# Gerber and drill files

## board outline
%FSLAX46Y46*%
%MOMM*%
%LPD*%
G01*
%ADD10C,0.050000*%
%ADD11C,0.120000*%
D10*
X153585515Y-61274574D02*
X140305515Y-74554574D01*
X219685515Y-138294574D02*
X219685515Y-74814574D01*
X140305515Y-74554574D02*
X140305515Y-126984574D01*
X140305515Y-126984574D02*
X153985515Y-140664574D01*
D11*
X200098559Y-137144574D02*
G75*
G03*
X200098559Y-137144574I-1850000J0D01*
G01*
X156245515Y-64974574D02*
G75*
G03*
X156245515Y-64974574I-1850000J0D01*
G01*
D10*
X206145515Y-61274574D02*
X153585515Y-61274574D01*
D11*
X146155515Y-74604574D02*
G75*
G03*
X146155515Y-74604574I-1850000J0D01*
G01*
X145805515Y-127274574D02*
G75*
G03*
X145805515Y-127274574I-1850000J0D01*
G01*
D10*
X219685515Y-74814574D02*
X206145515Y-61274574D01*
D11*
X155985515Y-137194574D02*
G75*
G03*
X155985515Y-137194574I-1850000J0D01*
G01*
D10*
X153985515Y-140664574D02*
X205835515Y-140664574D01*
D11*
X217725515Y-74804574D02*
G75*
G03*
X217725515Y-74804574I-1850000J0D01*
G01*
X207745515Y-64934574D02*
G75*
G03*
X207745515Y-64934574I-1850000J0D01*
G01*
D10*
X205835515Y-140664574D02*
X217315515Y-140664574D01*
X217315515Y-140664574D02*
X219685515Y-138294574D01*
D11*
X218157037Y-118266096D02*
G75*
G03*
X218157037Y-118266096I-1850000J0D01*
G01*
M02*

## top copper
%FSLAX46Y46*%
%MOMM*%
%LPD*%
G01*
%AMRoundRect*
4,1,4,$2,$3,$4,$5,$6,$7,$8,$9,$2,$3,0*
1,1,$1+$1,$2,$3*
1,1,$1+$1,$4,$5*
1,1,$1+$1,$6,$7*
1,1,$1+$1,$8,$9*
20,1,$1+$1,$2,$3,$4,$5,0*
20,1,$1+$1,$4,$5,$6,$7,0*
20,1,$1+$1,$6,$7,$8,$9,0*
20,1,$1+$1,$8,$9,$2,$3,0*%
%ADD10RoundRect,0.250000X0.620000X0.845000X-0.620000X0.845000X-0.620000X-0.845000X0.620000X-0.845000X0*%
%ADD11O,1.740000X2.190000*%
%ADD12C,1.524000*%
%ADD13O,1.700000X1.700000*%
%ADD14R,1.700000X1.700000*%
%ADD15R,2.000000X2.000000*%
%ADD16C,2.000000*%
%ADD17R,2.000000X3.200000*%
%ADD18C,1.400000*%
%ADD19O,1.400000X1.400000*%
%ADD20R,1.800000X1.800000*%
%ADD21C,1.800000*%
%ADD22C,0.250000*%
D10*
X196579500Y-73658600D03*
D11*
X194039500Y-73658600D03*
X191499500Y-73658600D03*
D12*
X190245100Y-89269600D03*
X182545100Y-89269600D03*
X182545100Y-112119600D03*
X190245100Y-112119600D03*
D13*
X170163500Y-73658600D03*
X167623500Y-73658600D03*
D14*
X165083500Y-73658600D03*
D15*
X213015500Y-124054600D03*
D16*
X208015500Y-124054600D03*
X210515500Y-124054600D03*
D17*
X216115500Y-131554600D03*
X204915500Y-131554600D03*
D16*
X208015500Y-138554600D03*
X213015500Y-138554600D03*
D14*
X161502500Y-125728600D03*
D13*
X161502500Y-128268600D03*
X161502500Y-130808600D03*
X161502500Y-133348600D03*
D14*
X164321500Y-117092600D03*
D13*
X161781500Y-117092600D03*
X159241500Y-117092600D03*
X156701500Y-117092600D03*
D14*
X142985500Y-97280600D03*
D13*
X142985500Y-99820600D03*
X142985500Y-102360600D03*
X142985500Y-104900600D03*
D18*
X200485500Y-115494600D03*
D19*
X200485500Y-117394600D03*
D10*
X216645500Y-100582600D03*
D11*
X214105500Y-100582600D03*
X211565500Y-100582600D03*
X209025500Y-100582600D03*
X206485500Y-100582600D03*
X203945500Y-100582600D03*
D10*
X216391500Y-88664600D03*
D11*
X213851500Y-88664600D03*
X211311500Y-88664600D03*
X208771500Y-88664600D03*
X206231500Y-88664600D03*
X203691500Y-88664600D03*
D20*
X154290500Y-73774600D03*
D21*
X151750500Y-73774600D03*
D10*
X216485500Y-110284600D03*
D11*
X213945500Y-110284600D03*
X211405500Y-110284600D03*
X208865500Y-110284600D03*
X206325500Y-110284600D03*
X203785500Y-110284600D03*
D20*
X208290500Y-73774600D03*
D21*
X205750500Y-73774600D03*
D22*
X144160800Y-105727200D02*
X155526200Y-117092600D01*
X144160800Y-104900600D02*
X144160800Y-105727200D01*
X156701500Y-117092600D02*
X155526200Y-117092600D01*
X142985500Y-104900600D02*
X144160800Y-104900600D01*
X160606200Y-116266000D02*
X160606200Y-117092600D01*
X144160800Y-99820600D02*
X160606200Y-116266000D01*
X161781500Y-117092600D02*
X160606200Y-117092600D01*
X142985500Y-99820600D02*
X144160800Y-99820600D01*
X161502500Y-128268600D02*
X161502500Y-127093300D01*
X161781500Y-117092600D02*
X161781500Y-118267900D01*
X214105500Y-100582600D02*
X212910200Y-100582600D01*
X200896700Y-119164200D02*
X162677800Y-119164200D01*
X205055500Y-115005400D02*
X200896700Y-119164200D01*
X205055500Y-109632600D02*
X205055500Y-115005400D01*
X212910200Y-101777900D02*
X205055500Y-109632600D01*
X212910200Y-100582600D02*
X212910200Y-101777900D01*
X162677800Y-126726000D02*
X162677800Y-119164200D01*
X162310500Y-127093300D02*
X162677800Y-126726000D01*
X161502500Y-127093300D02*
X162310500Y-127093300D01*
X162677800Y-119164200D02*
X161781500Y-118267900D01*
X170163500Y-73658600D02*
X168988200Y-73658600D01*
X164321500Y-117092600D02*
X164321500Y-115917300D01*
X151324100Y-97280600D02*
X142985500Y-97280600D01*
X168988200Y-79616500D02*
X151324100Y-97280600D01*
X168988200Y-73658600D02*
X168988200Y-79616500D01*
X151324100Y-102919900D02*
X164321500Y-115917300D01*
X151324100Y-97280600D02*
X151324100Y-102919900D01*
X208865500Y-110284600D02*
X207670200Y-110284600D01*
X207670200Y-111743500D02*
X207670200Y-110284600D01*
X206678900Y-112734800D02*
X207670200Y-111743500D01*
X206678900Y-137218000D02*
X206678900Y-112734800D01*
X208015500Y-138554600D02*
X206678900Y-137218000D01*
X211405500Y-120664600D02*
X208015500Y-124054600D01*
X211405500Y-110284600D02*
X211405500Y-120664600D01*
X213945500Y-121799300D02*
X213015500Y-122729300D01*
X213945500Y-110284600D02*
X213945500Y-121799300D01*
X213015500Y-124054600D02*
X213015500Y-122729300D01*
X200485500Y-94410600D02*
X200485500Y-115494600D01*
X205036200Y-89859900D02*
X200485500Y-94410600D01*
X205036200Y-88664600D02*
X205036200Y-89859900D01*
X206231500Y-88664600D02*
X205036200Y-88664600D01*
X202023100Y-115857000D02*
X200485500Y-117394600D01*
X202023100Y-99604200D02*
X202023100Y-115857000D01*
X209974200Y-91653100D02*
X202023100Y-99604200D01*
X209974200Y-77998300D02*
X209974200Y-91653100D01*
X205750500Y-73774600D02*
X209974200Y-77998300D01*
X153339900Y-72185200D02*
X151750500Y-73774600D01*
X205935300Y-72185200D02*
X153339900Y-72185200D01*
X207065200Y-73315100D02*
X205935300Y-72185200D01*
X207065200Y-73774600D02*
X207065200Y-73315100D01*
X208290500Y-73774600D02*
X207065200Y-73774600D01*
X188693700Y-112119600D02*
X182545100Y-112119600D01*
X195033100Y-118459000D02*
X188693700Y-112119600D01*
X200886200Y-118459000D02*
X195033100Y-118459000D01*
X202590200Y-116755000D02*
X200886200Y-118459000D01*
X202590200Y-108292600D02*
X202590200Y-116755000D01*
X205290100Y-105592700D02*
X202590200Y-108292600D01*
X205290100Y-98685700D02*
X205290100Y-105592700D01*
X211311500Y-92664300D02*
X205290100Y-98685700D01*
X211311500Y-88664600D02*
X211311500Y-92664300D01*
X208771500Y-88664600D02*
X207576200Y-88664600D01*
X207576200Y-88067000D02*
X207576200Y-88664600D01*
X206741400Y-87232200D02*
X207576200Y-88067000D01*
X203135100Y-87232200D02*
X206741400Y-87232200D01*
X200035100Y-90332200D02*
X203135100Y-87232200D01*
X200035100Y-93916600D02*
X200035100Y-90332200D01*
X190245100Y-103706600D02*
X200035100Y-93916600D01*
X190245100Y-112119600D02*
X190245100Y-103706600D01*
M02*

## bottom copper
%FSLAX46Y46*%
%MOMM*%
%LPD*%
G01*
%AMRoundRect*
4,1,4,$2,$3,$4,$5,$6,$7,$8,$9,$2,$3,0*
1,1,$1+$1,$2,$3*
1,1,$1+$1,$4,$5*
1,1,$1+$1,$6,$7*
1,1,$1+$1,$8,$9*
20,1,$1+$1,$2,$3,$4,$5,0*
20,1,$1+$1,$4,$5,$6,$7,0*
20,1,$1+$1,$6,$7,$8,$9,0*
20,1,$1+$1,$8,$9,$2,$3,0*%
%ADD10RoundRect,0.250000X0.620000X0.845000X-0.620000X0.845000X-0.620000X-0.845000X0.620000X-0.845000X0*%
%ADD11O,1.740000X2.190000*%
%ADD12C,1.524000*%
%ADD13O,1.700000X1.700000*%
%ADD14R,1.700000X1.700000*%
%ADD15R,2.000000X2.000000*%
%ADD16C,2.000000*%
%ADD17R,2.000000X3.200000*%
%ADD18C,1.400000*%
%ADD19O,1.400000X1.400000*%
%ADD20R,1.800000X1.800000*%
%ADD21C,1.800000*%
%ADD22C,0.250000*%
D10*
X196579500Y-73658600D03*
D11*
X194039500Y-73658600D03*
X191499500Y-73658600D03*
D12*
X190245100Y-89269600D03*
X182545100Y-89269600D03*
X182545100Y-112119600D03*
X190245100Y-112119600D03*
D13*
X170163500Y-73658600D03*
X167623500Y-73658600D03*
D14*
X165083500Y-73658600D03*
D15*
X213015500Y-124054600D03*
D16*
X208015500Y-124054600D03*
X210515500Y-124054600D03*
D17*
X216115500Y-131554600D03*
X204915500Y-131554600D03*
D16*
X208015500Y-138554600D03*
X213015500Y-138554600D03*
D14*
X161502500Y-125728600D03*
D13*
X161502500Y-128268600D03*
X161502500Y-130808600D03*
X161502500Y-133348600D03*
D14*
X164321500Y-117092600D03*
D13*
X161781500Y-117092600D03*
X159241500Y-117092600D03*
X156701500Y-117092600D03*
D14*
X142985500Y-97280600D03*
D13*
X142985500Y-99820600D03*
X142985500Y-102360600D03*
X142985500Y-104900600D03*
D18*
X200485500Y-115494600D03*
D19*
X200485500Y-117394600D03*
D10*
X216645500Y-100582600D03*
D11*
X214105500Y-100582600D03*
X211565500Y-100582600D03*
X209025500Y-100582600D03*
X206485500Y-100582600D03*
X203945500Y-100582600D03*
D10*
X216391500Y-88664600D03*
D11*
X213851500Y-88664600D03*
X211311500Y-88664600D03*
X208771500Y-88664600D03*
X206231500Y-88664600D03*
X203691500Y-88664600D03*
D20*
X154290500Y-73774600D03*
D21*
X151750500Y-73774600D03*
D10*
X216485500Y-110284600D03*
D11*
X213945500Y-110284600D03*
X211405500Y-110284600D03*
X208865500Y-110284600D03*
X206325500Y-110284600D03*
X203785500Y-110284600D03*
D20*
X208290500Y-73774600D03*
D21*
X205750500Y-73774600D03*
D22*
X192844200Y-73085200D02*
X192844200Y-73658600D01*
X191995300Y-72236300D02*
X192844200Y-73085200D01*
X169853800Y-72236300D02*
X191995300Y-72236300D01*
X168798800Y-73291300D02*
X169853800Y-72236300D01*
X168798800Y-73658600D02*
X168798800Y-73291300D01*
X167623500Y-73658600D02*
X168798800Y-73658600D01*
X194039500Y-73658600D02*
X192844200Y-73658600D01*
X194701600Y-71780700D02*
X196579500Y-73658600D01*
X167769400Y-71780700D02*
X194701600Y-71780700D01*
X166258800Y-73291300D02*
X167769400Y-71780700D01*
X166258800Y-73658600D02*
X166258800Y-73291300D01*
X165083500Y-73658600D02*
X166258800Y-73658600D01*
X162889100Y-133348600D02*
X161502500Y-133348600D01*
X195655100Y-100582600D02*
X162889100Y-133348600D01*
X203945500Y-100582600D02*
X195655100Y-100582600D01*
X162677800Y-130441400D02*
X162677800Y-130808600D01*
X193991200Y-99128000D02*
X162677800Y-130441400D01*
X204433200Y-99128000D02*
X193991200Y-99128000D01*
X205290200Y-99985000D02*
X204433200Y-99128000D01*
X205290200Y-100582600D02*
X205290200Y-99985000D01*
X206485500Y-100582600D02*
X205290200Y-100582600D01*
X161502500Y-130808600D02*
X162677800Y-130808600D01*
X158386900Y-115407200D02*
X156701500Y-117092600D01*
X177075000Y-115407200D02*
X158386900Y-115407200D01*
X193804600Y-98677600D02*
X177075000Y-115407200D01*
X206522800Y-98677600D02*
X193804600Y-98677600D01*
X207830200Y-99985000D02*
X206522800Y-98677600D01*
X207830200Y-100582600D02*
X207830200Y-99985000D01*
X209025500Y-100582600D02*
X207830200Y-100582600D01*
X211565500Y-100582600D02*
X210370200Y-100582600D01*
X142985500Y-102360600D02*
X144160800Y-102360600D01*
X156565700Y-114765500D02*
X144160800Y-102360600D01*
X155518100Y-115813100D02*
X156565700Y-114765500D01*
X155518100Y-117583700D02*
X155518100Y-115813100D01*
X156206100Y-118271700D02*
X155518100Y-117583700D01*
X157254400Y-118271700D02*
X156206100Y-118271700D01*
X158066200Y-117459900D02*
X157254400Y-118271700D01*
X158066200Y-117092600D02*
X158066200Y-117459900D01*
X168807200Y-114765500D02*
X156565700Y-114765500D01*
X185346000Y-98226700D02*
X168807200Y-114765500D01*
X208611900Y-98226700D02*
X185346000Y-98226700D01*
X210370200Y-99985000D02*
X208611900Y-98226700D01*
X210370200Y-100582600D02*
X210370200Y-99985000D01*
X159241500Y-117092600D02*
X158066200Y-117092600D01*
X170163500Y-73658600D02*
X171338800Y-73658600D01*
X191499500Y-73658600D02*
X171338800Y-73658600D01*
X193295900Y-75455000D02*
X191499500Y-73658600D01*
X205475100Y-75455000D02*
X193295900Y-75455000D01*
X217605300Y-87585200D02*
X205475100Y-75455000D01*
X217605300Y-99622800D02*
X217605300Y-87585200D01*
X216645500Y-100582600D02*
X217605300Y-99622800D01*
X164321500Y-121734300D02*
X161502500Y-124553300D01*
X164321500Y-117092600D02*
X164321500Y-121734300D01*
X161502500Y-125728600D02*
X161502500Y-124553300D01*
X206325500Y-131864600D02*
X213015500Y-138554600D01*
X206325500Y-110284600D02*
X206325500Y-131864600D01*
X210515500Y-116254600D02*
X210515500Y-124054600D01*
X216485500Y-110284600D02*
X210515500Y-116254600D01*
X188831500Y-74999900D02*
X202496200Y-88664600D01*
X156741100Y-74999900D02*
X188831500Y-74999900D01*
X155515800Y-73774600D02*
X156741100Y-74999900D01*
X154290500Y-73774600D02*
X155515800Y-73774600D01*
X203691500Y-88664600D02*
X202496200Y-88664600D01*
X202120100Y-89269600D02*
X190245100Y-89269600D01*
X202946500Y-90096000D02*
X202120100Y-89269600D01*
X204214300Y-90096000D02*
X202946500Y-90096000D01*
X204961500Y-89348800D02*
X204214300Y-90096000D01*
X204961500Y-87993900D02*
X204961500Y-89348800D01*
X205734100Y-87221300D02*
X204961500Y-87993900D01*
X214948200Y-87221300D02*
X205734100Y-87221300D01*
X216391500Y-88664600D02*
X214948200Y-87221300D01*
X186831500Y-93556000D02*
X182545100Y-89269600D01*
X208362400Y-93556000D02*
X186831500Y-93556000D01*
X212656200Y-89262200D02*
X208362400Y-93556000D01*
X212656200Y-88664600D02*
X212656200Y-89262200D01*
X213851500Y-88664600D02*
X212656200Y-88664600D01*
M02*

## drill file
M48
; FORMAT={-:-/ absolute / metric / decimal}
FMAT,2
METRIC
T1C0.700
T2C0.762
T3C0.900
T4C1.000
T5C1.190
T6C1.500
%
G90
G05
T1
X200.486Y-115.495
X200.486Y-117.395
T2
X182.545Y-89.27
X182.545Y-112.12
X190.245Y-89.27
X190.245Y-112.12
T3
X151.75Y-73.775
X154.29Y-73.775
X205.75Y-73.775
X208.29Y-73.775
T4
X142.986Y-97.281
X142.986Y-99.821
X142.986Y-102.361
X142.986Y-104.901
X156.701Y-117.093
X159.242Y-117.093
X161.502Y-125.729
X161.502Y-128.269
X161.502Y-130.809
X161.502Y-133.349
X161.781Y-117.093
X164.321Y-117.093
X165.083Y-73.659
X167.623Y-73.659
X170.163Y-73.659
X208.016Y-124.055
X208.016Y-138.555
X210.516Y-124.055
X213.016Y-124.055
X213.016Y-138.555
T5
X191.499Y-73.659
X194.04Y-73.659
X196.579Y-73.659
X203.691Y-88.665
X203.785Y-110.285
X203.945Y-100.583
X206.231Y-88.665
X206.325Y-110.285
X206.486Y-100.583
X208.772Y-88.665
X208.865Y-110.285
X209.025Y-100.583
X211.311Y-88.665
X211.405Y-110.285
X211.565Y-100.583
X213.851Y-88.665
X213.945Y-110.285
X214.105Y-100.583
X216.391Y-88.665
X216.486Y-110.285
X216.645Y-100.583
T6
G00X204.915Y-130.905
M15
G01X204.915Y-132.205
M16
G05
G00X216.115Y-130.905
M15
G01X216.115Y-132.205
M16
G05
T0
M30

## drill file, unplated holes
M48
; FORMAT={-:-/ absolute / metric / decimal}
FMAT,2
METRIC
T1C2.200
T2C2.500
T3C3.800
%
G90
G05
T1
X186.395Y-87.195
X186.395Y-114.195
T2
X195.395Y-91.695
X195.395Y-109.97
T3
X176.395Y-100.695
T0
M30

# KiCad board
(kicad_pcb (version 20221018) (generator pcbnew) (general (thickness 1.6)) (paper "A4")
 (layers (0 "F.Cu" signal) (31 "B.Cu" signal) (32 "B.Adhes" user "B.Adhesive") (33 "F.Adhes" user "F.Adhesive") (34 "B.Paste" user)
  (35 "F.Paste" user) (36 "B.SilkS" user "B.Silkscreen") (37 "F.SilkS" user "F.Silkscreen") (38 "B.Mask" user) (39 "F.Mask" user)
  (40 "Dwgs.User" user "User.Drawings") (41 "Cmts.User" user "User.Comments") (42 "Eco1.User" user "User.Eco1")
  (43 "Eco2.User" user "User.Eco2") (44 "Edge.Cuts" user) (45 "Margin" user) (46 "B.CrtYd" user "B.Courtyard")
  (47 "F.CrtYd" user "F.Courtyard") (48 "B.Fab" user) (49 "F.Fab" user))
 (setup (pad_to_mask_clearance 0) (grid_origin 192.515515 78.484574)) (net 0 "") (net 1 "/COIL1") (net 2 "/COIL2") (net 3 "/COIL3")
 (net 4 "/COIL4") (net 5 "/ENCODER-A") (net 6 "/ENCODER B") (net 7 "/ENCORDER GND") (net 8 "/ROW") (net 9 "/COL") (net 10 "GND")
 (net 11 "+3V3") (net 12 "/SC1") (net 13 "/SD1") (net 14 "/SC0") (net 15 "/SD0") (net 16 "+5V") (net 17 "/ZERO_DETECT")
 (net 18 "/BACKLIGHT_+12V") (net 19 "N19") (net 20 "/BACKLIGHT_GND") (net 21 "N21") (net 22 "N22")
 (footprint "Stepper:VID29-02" (layer "F.Cu") (at 186.3951 100.8596 -90)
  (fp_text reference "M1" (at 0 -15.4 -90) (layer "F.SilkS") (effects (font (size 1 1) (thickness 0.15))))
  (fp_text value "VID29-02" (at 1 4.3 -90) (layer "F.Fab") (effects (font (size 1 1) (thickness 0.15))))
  (pad "" np_thru_hole circle (at -13.665 0 270) (size 2.2 2.2) (drill 2.2) (layers "*.Cu" "*.Mask"))
  (pad "" np_thru_hole circle (at -9.165 -9 270) (size 2.5 2.5) (drill 2.5) (layers "*.Cu" "*.Mask"))
  (pad "" np_thru_hole circle (at -0.165 10 270) (size 3.8 3.8) (drill 3.8) (layers "*.Cu" "*.Mask"))
  (pad "" np_thru_hole circle (at 9.11 -9 270) (size 2.5 2.5) (drill 2.5) (layers "*.Cu" "*.Mask"))
  (pad "" np_thru_hole circle (at 13.335 0 270) (size 2.2 2.2) (drill 2.2) (layers "*.Cu" "*.Mask"))
  (pad "1" thru_hole circle (at -11.59 -3.85 270) (size 1.524 1.524) (drill 0.762) (layers "*.Cu" "*.Mask") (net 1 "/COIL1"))
  (pad "2" thru_hole circle (at -11.59 3.85 270) (size 1.524 1.524) (drill 0.762) (layers "*.Cu" "*.Mask") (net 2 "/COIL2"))
  (pad "3" thru_hole circle (at 11.26 3.85 270) (size 1.524 1.524) (drill 0.762) (layers "*.Cu" "*.Mask") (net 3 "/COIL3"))
  (pad "4" thru_hole circle (at 11.26 -3.85 270) (size 1.524 1.524) (drill 0.762) (layers "*.Cu" "*.Mask") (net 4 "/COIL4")))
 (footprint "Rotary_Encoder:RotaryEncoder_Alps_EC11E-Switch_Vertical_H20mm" (layer "F.Cu") (at 213.0155 124.0546 -90)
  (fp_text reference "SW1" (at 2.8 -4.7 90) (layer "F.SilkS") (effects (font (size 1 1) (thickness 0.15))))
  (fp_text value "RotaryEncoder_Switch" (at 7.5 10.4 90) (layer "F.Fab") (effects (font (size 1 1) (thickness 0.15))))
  (pad "A" thru_hole rect (at 0 0 270) (size 2 2) (drill 1) (layers "*.Cu" "*.Mask") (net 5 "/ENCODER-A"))
  (pad "B" thru_hole circle (at 0 5 270) (size 2 2) (drill 1) (layers "*.Cu" "*.Mask") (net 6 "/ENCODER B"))
  (pad "C" thru_hole circle (at 0 2.5 270) (size 2 2) (drill 1) (layers "*.Cu" "*.Mask") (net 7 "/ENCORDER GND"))
  (pad "MP" thru_hole rect (at 7.5 -3.1 270) (size 3.2 2) (drill oval 2.8 1.5) (layers "*.Cu" "*.Mask"))
  (pad "MP" thru_hole rect (at 7.5 8.1 270) (size 3.2 2) (drill oval 2.8 1.5) (layers "*.Cu" "*.Mask"))
  (pad "S1" thru_hole circle (at 14.5 5 270) (size 2 2) (drill 1) (layers "*.Cu" "*.Mask") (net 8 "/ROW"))
  (pad "S2" thru_hole circle (at 14.5 0 270) (size 2 2) (drill 1) (layers "*.Cu" "*.Mask") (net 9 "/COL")))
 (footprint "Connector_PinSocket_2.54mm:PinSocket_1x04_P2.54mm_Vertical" (layer "F.Cu") (at 161.5025 125.7286)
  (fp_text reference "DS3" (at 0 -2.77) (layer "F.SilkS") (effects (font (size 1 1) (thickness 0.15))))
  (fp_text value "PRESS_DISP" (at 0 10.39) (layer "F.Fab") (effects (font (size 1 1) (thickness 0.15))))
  (pad "1" thru_hole rect (at 0 0) (size 1.7 1.7) (drill 1) (layers "*.Cu" "*.Mask") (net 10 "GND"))
  (pad "2" thru_hole oval (at 0 2.54) (size 1.7 1.7) (drill 1) (layers "*.Cu" "*.Mask") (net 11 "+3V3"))
  (pad "3" thru_hole oval (at 0 5.08) (size 1.7 1.7) (drill 1) (layers "*.Cu" "*.Mask") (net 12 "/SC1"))
  (pad "4" thru_hole oval (at 0 7.62) (size 1.7 1.7) (drill 1) (layers "*.Cu" "*.Mask") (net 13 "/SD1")))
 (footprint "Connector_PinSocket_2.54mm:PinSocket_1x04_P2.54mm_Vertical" (layer "F.Cu") (at 164.3215 117.0926 -90)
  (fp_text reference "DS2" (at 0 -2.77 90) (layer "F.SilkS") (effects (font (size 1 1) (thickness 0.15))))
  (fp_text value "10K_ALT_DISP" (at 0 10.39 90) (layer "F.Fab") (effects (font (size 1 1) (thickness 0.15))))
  (pad "1" thru_hole rect (at 0 0 270) (size 1.7 1.7) (drill 1) (layers "*.Cu" "*.Mask") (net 10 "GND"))
  (pad "2" thru_hole oval (at 0 2.54 270) (size 1.7 1.7) (drill 1) (layers "*.Cu" "*.Mask") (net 11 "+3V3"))
  (pad "3" thru_hole oval (at 0 5.08 270) (size 1.7 1.7) (drill 1) (layers "*.Cu" "*.Mask") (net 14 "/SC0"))
  (pad "4" thru_hole oval (at 0 7.62 270) (size 1.7 1.7) (drill 1) (layers "*.Cu" "*.Mask") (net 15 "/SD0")))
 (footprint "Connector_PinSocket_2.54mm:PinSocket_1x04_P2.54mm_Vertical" (layer "F.Cu") (at 142.9855 97.2806)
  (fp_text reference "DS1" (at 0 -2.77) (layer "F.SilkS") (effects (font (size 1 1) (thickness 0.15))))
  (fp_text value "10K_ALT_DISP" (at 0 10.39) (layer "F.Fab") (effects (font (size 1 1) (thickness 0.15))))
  (pad "1" thru_hole rect (at 0 0) (size 1.7 1.7) (drill 1) (layers "*.Cu" "*.Mask") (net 10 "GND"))
  (pad "2" thru_hole oval (at 0 2.54) (size 1.7 1.7) (drill 1) (layers "*.Cu" "*.Mask") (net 11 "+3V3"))
  (pad "3" thru_hole oval (at 0 5.08) (size 1.7 1.7) (drill 1) (layers "*.Cu" "*.Mask") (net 14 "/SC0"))
  (pad "4" thru_hole oval (at 0 7.62) (size 1.7 1.7) (drill 1) (layers "*.Cu" "*.Mask") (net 15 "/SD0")))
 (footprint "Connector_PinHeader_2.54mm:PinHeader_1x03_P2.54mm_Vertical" (layer "B.Cu") (at 165.0835 73.6586 -90)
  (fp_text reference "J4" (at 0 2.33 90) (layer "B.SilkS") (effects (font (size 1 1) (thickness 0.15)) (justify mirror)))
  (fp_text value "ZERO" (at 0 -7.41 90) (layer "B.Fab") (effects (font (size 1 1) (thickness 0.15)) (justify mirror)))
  (pad "1" thru_hole rect (at 0 0 270) (size 1.7 1.7) (drill 1) (layers "*.Cu" "*.Mask") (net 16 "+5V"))
  (pad "2" thru_hole oval (at 0 -2.54 270) (size 1.7 1.7) (drill 1) (layers "*.Cu" "*.Mask") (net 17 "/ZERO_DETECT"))
  (pad "3" thru_hole oval (at 0 -5.08 270) (size 1.7 1.7) (drill 1) (layers "*.Cu" "*.Mask") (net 10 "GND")))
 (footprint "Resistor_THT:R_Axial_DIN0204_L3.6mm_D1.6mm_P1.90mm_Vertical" (layer "B.Cu") (at 200.4855 115.4946 -90)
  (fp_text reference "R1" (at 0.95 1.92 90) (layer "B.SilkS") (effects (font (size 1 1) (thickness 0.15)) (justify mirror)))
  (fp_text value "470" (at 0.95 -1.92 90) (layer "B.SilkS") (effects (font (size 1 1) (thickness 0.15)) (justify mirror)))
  (pad "1" thru_hole circle (at 0 0 270) (size 1.4 1.4) (drill 0.7) (layers "*.Cu" "*.Mask") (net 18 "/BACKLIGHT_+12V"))
  (pad "2" thru_hole oval (at 1.9 0 270) (size 1.4 1.4) (drill 0.7) (layers "*.Cu" "*.Mask") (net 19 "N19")))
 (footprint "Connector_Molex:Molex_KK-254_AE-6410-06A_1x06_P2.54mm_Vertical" (layer "B.Cu") (at 216.6455 100.5826 180)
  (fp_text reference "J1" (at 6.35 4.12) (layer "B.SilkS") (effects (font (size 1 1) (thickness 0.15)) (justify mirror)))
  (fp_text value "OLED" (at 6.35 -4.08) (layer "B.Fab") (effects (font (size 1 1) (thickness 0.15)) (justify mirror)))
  (pad "1" thru_hole roundrect (at 0 0 180) (size 1.74 2.19) (drill 1.19) (layers "*.Cu" "*.Mask") (roundrect_rratio 0.1436781609)
   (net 10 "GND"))
  (pad "2" thru_hole oval (at 2.54 0 180) (size 1.74 2.19) (drill 1.19) (layers "*.Cu" "*.Mask") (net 11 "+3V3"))
  (pad "3" thru_hole oval (at 5.08 0 180) (size 1.74 2.19) (drill 1.19) (layers "*.Cu" "*.Mask") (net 14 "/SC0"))
  (pad "4" thru_hole oval (at 7.62 0 180) (size 1.74 2.19) (drill 1.19) (layers "*.Cu" "*.Mask") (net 15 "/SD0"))
  (pad "5" thru_hole oval (at 10.16 0 180) (size 1.74 2.19) (drill 1.19) (layers "*.Cu" "*.Mask") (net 12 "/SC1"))
  (pad "6" thru_hole oval (at 12.7 0 180) (size 1.74 2.19) (drill 1.19) (layers "*.Cu" "*.Mask") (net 13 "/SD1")))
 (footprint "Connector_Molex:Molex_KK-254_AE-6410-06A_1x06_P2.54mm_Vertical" (layer "B.Cu") (at 216.3915 88.6646 180)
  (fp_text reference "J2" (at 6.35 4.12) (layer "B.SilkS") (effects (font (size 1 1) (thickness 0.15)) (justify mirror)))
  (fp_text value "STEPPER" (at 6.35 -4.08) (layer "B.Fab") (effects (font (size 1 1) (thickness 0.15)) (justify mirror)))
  (pad "1" thru_hole roundrect (at 0 0 180) (size 1.74 2.19) (drill 1.19) (layers "*.Cu" "*.Mask") (roundrect_rratio 0.1436781609)
   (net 1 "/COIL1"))
  (pad "2" thru_hole oval (at 2.54 0 180) (size 1.74 2.19) (drill 1.19) (layers "*.Cu" "*.Mask") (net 2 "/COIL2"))
  (pad "3" thru_hole oval (at 5.08 0 180) (size 1.74 2.19) (drill 1.19) (layers "*.Cu" "*.Mask") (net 3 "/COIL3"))
  (pad "4" thru_hole oval (at 7.62 0 180) (size 1.74 2.19) (drill 1.19) (layers "*.Cu" "*.Mask") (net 4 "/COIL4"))
  (pad "5" thru_hole oval (at 10.16 0 180) (size 1.74 2.19) (drill 1.19) (layers "*.Cu" "*.Mask") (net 18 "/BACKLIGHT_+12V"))
  (pad "6" thru_hole oval (at 12.7 0 180) (size 1.74 2.19) (drill 1.19) (layers "*.Cu" "*.Mask") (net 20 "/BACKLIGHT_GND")))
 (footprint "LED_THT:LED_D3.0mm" (layer "B.Cu") (at 154.2905 73.7746 180)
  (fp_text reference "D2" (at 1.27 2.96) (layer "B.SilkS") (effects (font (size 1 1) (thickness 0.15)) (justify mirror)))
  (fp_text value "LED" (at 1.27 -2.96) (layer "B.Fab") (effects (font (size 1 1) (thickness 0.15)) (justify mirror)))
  (pad "1" thru_hole rect (at 0 0 180) (size 1.8 1.8) (drill 0.9) (layers "*.Cu" "*.Mask") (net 20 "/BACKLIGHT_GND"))
  (pad "2" thru_hole circle (at 2.54 0 180) (size 1.8 1.8) (drill 0.9) (layers "*.Cu" "*.Mask") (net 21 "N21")))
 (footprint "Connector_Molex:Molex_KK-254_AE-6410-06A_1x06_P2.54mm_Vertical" (layer "B.Cu") (at 216.4855 110.2846 180)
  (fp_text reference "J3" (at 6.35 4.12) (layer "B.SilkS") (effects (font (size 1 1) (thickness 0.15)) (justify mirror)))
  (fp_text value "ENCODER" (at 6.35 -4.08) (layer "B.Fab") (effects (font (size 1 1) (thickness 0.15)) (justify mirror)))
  (pad "1" thru_hole roundrect (at 0 0 180) (size 1.74 2.19) (drill 1.19) (layers "*.Cu" "*.Mask") (roundrect_rratio 0.1436781609)
   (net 7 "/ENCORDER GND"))
  (pad "2" thru_hole oval (at 2.54 0 180) (size 1.74 2.19) (drill 1.19) (layers "*.Cu" "*.Mask") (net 5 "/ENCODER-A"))
  (pad "3" thru_hole oval (at 5.08 0 180) (size 1.74 2.19) (drill 1.19) (layers "*.Cu" "*.Mask") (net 6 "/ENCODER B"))
  (pad "4" thru_hole oval (at 7.62 0 180) (size 1.74 2.19) (drill 1.19) (layers "*.Cu" "*.Mask") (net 8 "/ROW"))
  (pad "5" thru_hole oval (at 10.16 0 180) (size 1.74 2.19) (drill 1.19) (layers "*.Cu" "*.Mask") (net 9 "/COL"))
  (pad "6" thru_hole oval (at 12.7 0 180) (size 1.74 2.19) (drill 1.19) (layers "*.Cu" "*.Mask") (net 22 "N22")))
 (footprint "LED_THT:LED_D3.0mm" (layer "B.Cu") (at 208.2905 73.7746 180)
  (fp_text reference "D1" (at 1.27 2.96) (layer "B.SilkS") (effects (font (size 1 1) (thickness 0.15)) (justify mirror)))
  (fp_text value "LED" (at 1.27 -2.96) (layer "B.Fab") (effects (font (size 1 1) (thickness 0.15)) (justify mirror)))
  (pad "1" thru_hole rect (at 0 0 180) (size 1.8 1.8) (drill 0.9) (layers "*.Cu" "*.Mask") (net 21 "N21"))
  (pad "2" thru_hole circle (at 2.54 0 180) (size 1.8 1.8) (drill 0.9) (layers "*.Cu" "*.Mask") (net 19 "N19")))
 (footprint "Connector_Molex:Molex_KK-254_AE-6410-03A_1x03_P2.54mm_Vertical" (layer "B.Cu") (at 196.5795 73.6586 180)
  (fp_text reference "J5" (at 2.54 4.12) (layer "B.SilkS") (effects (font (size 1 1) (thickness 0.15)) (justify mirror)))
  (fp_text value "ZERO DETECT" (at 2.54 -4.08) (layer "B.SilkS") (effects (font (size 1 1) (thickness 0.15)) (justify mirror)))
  (pad "1" thru_hole roundrect (at 0 0 180) (size 1.74 2.19) (drill 1.19) (layers "*.Cu" "*.Mask") (roundrect_rratio 0.1436781609)
   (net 16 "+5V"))
  (pad "2" thru_hole oval (at 2.54 0 180) (size 1.74 2.19) (drill 1.19) (layers "*.Cu" "*.Mask") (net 17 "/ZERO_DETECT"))
  (pad "3" thru_hole oval (at 5.08 0 180) (size 1.74 2.19) (drill 1.19) (layers "*.Cu" "*.Mask") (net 10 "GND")))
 (gr_line (start 153.585515 61.274574) (end 140.305515 74.554574) (stroke (width 0.05) (type solid)) (layer "Edge.Cuts"))
 (gr_line (start 219.685515 138.294574) (end 219.685515 74.814574) (stroke (width 0.05) (type solid)) (layer "Edge.Cuts"))
 (gr_line (start 140.305515 74.554574) (end 140.305515 126.984574) (stroke (width 0.05) (type solid)) (layer "Edge.Cuts"))
 (gr_line (start 140.305515 126.984574) (end 153.985515 140.664574) (stroke (width 0.05) (type solid)) (layer "Edge.Cuts"))
 (gr_circle (center 198.248559 137.144574) (end 200.098559 137.144574) (stroke (width 0.12) (type solid)) (fill none) (layer "Edge.Cuts"))
 (gr_circle (center 154.395515 64.974574) (end 156.245515 64.974574) (stroke (width 0.12) (type solid)) (fill none) (layer "Edge.Cuts"))
 (gr_line (start 206.145515 61.274574) (end 153.585515 61.274574) (stroke (width 0.05) (type solid)) (layer "Edge.Cuts"))
 (gr_circle (center 144.305515 74.604574) (end 146.155515 74.604574) (stroke (width 0.12) (type solid)) (fill none) (layer "Edge.Cuts"))
 (gr_circle (center 143.955515 127.274574) (end 145.805515 127.274574) (stroke (width 0.12) (type solid)) (fill none) (layer "Edge.Cuts"))
 (gr_line (start 219.685515 74.814574) (end 206.145515 61.274574) (stroke (width 0.05) (type solid)) (layer "Edge.Cuts"))
 (gr_circle (center 154.135515 137.194574) (end 155.985515 137.194574) (stroke (width 0.12) (type solid)) (fill none) (layer "Edge.Cuts"))
 (gr_line (start 153.985515 140.664574) (end 205.835515 140.664574) (stroke (width 0.05) (type solid)) (layer "Edge.Cuts"))
 (gr_circle (center 215.875515 74.804574) (end 217.725515 74.804574) (stroke (width 0.12) (type solid)) (fill none) (layer "Edge.Cuts"))
 (gr_circle (center 205.895515 64.934574) (end 207.745515 64.934574) (stroke (width 0.12) (type solid)) (fill none) (layer "Edge.Cuts"))
 (gr_line (start 205.835515 140.664574) (end 217.315515 140.664574) (stroke (width 0.05) (type solid)) (layer "Edge.Cuts"))
 (gr_line (start 217.315515 140.664574) (end 219.685515 138.294574) (stroke (width 0.05) (type solid)) (layer "Edge.Cuts"))
 (gr_circle (center 216.307037 118.266096) (end 218.157037 118.266096) (stroke (width 0.12) (type solid)) (fill none) (layer "Edge.Cuts"))
 (segment (start 212.6562 89.2622) (end 208.3624 93.556) (width 0.25) (layer "B.Cu") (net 2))
 (segment (start 208.3624 93.556) (end 186.8315 93.556) (width 0.25) (layer "B.Cu") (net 2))
 (segment (start 213.8515 88.6646) (end 212.6562 88.6646) (width 0.25) (layer "B.Cu") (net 2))
 (segment (start 212.6562 88.6646) (end 212.6562 89.2622) (width 0.25) (layer "B.Cu") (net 2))
 (segment (start 186.8315 93.556) (end 182.5451 89.2696) (width 0.25) (layer "B.Cu") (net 2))
 (segment (start 202.1201 89.2696) (end 190.2451 89.2696) (width 0.25) (layer "B.Cu") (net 1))
 (segment (start 202.9465 90.096) (end 202.1201 89.2696) (width 0.25) (layer "B.Cu") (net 1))
 (segment (start 204.9615 89.3488) (end 204.2143 90.096) (width 0.25) (layer "B.Cu") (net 1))
 (segment (start 216.3915 88.6646) (end 214.9482 87.2213) (width 0.25) (layer "B.Cu") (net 1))
 (segment (start 204.2143 90.096) (end 202.9465 90.096) (width 0.25) (layer "B.Cu") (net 1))
 (segment (start 214.9482 87.2213) (end 205.7341 87.2213) (width 0.25) (layer "B.Cu") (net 1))
 (segment (start 204.9615 87.9939) (end 204.9615 89.3488) (width 0.25) (layer "B.Cu") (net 1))
 (segment (start 205.7341 87.2213) (end 204.9615 87.9939) (width 0.25) (layer "B.Cu") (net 1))
 (segment (start 190.2451 112.1196) (end 190.2451 103.7066) (width 0.25) (layer "F.Cu") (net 4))
 (segment (start 203.1351 87.2322) (end 206.7414 87.2322) (width 0.25) (layer "F.Cu") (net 4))
 (segment (start 200.0351 90.3322) (end 203.1351 87.2322) (width 0.25) (layer "F.Cu") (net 4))
 (segment (start 207.5762 88.067) (end 207.5762 88.6646) (width 0.25) (layer "F.Cu") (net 4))
 (segment (start 208.7715 88.6646) (end 207.5762 88.6646) (width 0.25) (layer "F.Cu") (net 4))
 (segment (start 190.2451 103.7066) (end 200.0351 93.9166) (width 0.25) (layer "F.Cu") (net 4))
 (segment (start 206.7414 87.2322) (end 207.5762 88.067) (width 0.25) (layer "F.Cu") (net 4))
 (segment (start 200.0351 93.9166) (end 200.0351 90.3322) (width 0.25) (layer "F.Cu") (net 4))
 (segment (start 205.2901 105.5927) (end 202.5902 108.2926) (width 0.25) (layer "F.Cu") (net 3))
 (segment (start 200.8862 118.459) (end 195.0331 118.459) (width 0.25) (layer "F.Cu") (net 3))
 (segment (start 211.3115 92.6643) (end 205.2901 98.6857) (width 0.25) (layer "F.Cu") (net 3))
 (segment (start 211.3115 88.6646) (end 211.3115 92.6643) (width 0.25) (layer "F.Cu") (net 3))
 (segment (start 202.5902 116.755) (end 200.8862 118.459) (width 0.25) (layer "F.Cu") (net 3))
 (segment (start 202.5902 108.2926) (end 202.5902 116.755) (width 0.25) (layer "F.Cu") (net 3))
 (segment (start 205.2901 98.6857) (end 205.2901 105.5927) (width 0.25) (layer "F.Cu") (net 3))
 (segment (start 188.6937 112.1196) (end 182.5451 112.1196) (width 0.25) (layer "F.Cu") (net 3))
 (segment (start 195.0331 118.459) (end 188.6937 112.1196) (width 0.25) (layer "F.Cu") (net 3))
 (segment (start 207.0652 73.3151) (end 205.9353 72.1852) (width 0.25) (layer "F.Cu") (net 21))
 (segment (start 153.3399 72.1852) (end 151.7505 73.7746) (width 0.25) (layer "F.Cu") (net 21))
 (segment (start 205.9353 72.1852) (end 153.3399 72.1852) (width 0.25) (layer "F.Cu") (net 21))
 (segment (start 208.2905 73.7746) (end 207.0652 73.7746) (width 0.25) (layer "F.Cu") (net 21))
 (segment (start 207.0652 73.7746) (end 207.0652 73.3151) (width 0.25) (layer "F.Cu") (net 21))
 (segment (start 209.9742 91.6531) (end 202.0231 99.6042) (width 0.25) (layer "F.Cu") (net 19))
 (segment (start 209.9742 77.9983) (end 209.9742 91.6531) (width 0.25) (layer "F.Cu") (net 19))
 (segment (start 202.0231 99.6042) (end 202.0231 115.857) (width 0.25) (layer "F.Cu") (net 19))
 (segment (start 202.0231 115.857) (end 200.4855 117.3946) (width 0.25) (layer "F.Cu") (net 19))
 (segment (start 205.7505 73.7746) (end 209.9742 77.9983) (width 0.25) (layer "F.Cu") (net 19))
 (segment (start 154.2905 73.7746) (end 155.5158 73.7746) (width 0.25) (layer "B.Cu") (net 20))
 (segment (start 156.7411 74.9999) (end 188.8315 74.9999) (width 0.25) (layer "B.Cu") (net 20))
 (segment (start 188.8315 74.9999) (end 202.4962 88.6646) (width 0.25) (layer "B.Cu") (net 20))
 (segment (start 203.6915 88.6646) (end 202.4962 88.6646) (width 0.25) (layer "B.Cu") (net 20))
 (segment (start 155.5158 73.7746) (end 156.7411 74.9999) (width 0.25) (layer "B.Cu") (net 20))
 (segment (start 200.4855 94.4106) (end 200.4855 115.4946) (width 0.25) (layer "F.Cu") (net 18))
 (segment (start 205.0362 89.8599) (end 200.4855 94.4106) (width 0.25) (layer "F.Cu") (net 18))
 (segment (start 206.2315 88.6646) (end 205.0362 88.6646) (width 0.25) (layer "F.Cu") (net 18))
 (segment (start 205.0362 88.6646) (end 205.0362 89.8599) (width 0.25) (layer "F.Cu") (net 18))
 (segment (start 216.4855 110.2846) (end 210.5155 116.2546) (width 0.25) (layer "B.Cu") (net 7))
 (segment (start 210.5155 116.2546) (end 210.5155 124.0546) (width 0.25) (layer "B.Cu") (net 7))
 (segment (start 213.9455 121.7993) (end 213.0155 122.7293) (width 0.25) (layer "F.Cu") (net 5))
 (segment (start 213.0155 124.0546) (end 213.0155 122.7293) (width 0.25) (layer "F.Cu") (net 5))
 (segment (start 213.9455 110.2846) (end 213.9455 121.7993) (width 0.25) (layer "F.Cu") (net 5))
 (segment (start 211.4055 110.2846) (end 211.4055 120.6646) (width 0.25) (layer "F.Cu") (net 6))
 (segment (start 211.4055 120.6646) (end 208.0155 124.0546) (width 0.25) (layer "F.Cu") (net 6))
 (segment (start 208.0155 138.5546) (end 206.6789 137.218) (width 0.25) (layer "F.Cu") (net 8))
 (segment (start 208.8655 110.2846) (end 207.6702 110.2846) (width 0.25) (layer "F.Cu") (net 8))
 (segment (start 206.6789 137.218) (end 206.6789 112.7348) (width 0.25) (layer "F.Cu") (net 8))
 (segment (start 207.6702 111.7435) (end 207.6702 110.2846) (width 0.25) (layer "F.Cu") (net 8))
 (segment (start 206.6789 112.7348) (end 207.6702 111.7435) (width 0.25) (layer "F.Cu") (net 8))
 (segment (start 206.3255 131.8646) (end 213.0155 138.5546) (width 0.25) (layer "B.Cu") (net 9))
 (segment (start 206.3255 110.2846) (end 206.3255 131.8646) (width 0.25) (layer "B.Cu") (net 9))
 (segment (start 168.9882 79.6165) (end 151.3241 97.2806) (width 0.25) (layer "F.Cu") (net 10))
 (segment (start 151.3241 97.2806) (end 151.3241 102.9199) (width 0.25) (layer "F.Cu") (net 10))
 (segment (start 170.1635 73.6586) (end 168.9882 73.6586) (width 0.25) (layer "F.Cu") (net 10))
 (segment (start 164.3215 117.0926) (end 164.3215 115.9173) (width 0.25) (layer "F.Cu") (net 10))
 (segment (start 151.3241 97.2806) (end 142.9855 97.2806) (width 0.25) (layer "F.Cu") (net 10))
 (segment (start 151.3241 102.9199) (end 164.3215 115.9173) (width 0.25) (layer "F.Cu") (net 10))
 (segment (start 168.9882 73.6586) (end 168.9882 79.6165) (width 0.25) (layer "F.Cu") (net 10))
 (segment (start 170.1635 73.6586) (end 171.3388 73.6586) (width 0.25) (layer "B.Cu") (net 10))
 (segment (start 164.3215 121.7343) (end 161.5025 124.5533) (width 0.25) (layer "B.Cu") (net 10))
 (segment (start 217.6053 87.5852) (end 205.4751 75.455) (width 0.25) (layer "B.Cu") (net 10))
 (segment (start 193.2959 75.455) (end 191.4995 73.6586) (width 0.25) (layer "B.Cu") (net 10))
 (segment (start 217.6053 99.6228) (end 217.6053 87.5852) (width 0.25) (layer "B.Cu") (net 10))
 (segment (start 205.4751 75.455) (end 193.2959 75.455) (width 0.25) (layer "B.Cu") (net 10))
 (segment (start 191.4995 73.6586) (end 171.3388 73.6586) (width 0.25) (layer "B.Cu") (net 10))
 (segment (start 216.6455 100.5826) (end 217.6053 99.6228) (width 0.25) (layer "B.Cu") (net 10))
 (segment (start 164.3215 117.0926) (end 164.3215 121.7343) (width 0.25) (layer "B.Cu") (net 10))
 (segment (start 161.5025 125.7286) (end 161.5025 124.5533) (width 0.25) (layer "B.Cu") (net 10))
 (segment (start 162.6778 119.1642) (end 161.7815 118.2679) (width 0.25) (layer "F.Cu") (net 11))
 (segment (start 161.7815 117.0926) (end 160.6062 117.0926) (width 0.25) (layer "F.Cu") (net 11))
 (segment (start 214.1055 100.5826) (end 212.9102 100.5826) (width 0.25) (layer "F.Cu") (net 11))
 (segment (start 144.1608 99.8206) (end 160.6062 116.266) (width 0.25) (layer "F.Cu") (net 11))
 (segment (start 162.3105 127.0933) (end 162.6778 126.726) (width 0.25) (layer "F.Cu") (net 11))
 (segment (start 212.9102 101.7779) (end 205.0555 109.6326) (width 0.25) (layer "F.Cu") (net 11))
 (segment (start 160.6062 116.266) (end 160.6062 117.0926) (width 0.25) (layer "F.Cu") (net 11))
 (segment (start 200.8967 119.1642) (end 162.6778 119.1642) (width 0.25) (layer "F.Cu") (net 11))
 (segment (start 205.0555 109.6326) (end 205.0555 115.0054) (width 0.25) (layer "F.Cu") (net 11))
 (segment (start 142.9855 99.8206) (end 144.1608 99.8206) (width 0.25) (layer "F.Cu") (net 11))
 (segment (start 212.9102 100.5826) (end 212.9102 101.7779) (width 0.25) (layer "F.Cu") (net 11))
 (segment (start 205.0555 115.0054) (end 200.8967 119.1642) (width 0.25) (layer "F.Cu") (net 11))
 (segment (start 161.5025 128.2686) (end 161.5025 127.0933) (width 0.25) (layer "F.Cu") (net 11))
 (segment (start 161.7815 117.0926) (end 161.7815 118.2679) (width 0.25) (layer "F.Cu") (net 11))
 (segment (start 162.6778 126.726) (end 162.6778 119.1642) (width 0.25) (layer "F.Cu") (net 11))
 (segment (start 161.5025 127.0933) (end 162.3105 127.0933) (width 0.25) (layer "F.Cu") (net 11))
 (segment (start 168.8072 114.7655) (end 156.5657 114.7655) (width 0.25) (layer "B.Cu") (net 14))
 (segment (start 185.346 98.2267) (end 168.8072 114.7655) (width 0.25) (layer "B.Cu") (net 14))
 (segment (start 159.2415 117.0926) (end 158.0662 117.0926) (width 0.25) (layer "B.Cu") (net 14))
 (segment (start 210.3702 100.5826) (end 210.3702 99.985) (width 0.25) (layer "B.Cu") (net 14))
 (segment (start 210.3702 99.985) (end 208.6119 98.2267) (width 0.25) (layer "B.Cu") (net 14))
 (segment (start 156.2061 118.2717) (end 155.5181 117.5837) (width 0.25) (layer "B.Cu") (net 14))
 (segment (start 158.0662 117.4599) (end 157.2544 118.2717) (width 0.25) (layer "B.Cu") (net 14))
 (segment (start 155.5181 117.5837) (end 155.5181 115.8131) (width 0.25) (layer "B.Cu") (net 14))
 (segment (start 211.5655 100.5826) (end 210.3702 100.5826) (width 0.25) (layer "B.Cu") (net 14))
 (segment (start 142.9855 102.3606) (end 144.1608 102.3606) (width 0.25) (layer "B.Cu") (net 14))
 (segment (start 156.5657 114.7655) (end 144.1608 102.3606) (width 0.25) (layer "B.Cu") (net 14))
 (segment (start 157.2544 118.2717) (end 156.2061 118.2717) (width 0.25) (layer "B.Cu") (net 14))
 (segment (start 208.6119 98.2267) (end 185.346 98.2267) (width 0.25) (layer "B.Cu") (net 14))
 (segment (start 155.5181 115.8131) (end 156.5657 114.7655) (width 0.25) (layer "B.Cu") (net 14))
 (segment (start 158.0662 117.0926) (end 158.0662 117.4599) (width 0.25) (layer "B.Cu") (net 14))
 (segment (start 142.9855 104.9006) (end 144.1608 104.9006) (width 0.25) (layer "F.Cu") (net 15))
 (segment (start 144.1608 105.7272) (end 155.5262 117.0926) (width 0.25) (layer "F.Cu") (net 15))
 (segment (start 144.1608 104.9006) (end 144.1608 105.7272) (width 0.25) (layer "F.Cu") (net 15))
 (segment (start 156.7015 117.0926) (end 155.5262 117.0926) (width 0.25) (layer "F.Cu") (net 15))
 (segment (start 158.3869 115.4072) (end 156.7015 117.0926) (width 0.25) (layer "B.Cu") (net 15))
 (segment (start 207.8302 99.985) (end 206.5228 98.6776) (width 0.25) (layer "B.Cu") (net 15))
 (segment (start 207.8302 100.5826) (end 207.8302 99.985) (width 0.25) (layer "B.Cu") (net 15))
 (segment (start 177.075 115.4072) (end 158.3869 115.4072) (width 0.25) (layer "B.Cu") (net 15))
 (segment (start 209.0255 100.5826) (end 207.8302 100.5826) (width 0.25) (layer "B.Cu") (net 15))
 (segment (start 206.5228 98.6776) (end 193.8046 98.6776) (width 0.25) (layer "B.Cu") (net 15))
 (segment (start 193.8046 98.6776) (end 177.075 115.4072) (width 0.25) (layer "B.Cu") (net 15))
 (segment (start 205.2902 100.5826) (end 205.2902 99.985) (width 0.25) (layer "B.Cu") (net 12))
 (segment (start 161.5025 130.8086) (end 162.6778 130.8086) (width 0.25) (layer "B.Cu") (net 12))
 (segment (start 162.6778 130.4414) (end 162.6778 130.8086) (width 0.25) (layer "B.Cu") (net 12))
 (segment (start 206.4855 100.5826) (end 205.2902 100.5826) (width 0.25) (layer "B.Cu") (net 12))
 (segment (start 204.4332 99.128) (end 193.9912 99.128) (width 0.25) (layer "B.Cu") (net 12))
 (segment (start 193.9912 99.128) (end 162.6778 130.4414) (width 0.25) (layer "B.Cu") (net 12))
 (segment (start 205.2902 99.985) (end 204.4332 99.128) (width 0.25) (layer "B.Cu") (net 12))
 (segment (start 195.6551 100.5826) (end 162.8891 133.3486) (width 0.25) (layer "B.Cu") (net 13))
 (segment (start 203.9455 100.5826) (end 195.6551 100.5826) (width 0.25) (layer "B.Cu") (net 13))
 (segment (start 162.8891 133.3486) (end 161.5025 133.3486) (width 0.25) (layer "B.Cu") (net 13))
 (segment (start 194.7016 71.7807) (end 196.5795 73.6586) (width 0.25) (layer "B.Cu") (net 16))
 (segment (start 167.7694 71.7807) (end 194.7016 71.7807) (width 0.25) (layer "B.Cu") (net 16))
 (segment (start 166.2588 73.2913) (end 167.7694 71.7807) (width 0.25) (layer "B.Cu") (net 16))
 (segment (start 166.2588 73.6586) (end 166.2588 73.2913) (width 0.25) (layer "B.Cu") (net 16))
 (segment (start 165.0835 73.6586) (end 166.2588 73.6586) (width 0.25) (layer "B.Cu") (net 16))
 (segment (start 191.9953 72.2363) (end 192.8442 73.0852) (width 0.25) (layer "B.Cu") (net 17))
 (segment (start 168.7988 73.2913) (end 169.8538 72.2363) (width 0.25) (layer "B.Cu") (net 17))
 (segment (start 169.8538 72.2363) (end 191.9953 72.2363) (width 0.25) (layer "B.Cu") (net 17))
 (segment (start 168.7988 73.6586) (end 168.7988 73.2913) (width 0.25) (layer "B.Cu") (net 17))
 (segment (start 194.0395 73.6586) (end 192.8442 73.6586) (width 0.25) (layer "B.Cu") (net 17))
 (segment (start 192.8442 73.0852) (end 192.8442 73.6586) (width 0.25) (layer "B.Cu") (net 17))
 (segment (start 167.6235 73.6586) (end 168.7988 73.6586) (width 0.25) (layer "B.Cu") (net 17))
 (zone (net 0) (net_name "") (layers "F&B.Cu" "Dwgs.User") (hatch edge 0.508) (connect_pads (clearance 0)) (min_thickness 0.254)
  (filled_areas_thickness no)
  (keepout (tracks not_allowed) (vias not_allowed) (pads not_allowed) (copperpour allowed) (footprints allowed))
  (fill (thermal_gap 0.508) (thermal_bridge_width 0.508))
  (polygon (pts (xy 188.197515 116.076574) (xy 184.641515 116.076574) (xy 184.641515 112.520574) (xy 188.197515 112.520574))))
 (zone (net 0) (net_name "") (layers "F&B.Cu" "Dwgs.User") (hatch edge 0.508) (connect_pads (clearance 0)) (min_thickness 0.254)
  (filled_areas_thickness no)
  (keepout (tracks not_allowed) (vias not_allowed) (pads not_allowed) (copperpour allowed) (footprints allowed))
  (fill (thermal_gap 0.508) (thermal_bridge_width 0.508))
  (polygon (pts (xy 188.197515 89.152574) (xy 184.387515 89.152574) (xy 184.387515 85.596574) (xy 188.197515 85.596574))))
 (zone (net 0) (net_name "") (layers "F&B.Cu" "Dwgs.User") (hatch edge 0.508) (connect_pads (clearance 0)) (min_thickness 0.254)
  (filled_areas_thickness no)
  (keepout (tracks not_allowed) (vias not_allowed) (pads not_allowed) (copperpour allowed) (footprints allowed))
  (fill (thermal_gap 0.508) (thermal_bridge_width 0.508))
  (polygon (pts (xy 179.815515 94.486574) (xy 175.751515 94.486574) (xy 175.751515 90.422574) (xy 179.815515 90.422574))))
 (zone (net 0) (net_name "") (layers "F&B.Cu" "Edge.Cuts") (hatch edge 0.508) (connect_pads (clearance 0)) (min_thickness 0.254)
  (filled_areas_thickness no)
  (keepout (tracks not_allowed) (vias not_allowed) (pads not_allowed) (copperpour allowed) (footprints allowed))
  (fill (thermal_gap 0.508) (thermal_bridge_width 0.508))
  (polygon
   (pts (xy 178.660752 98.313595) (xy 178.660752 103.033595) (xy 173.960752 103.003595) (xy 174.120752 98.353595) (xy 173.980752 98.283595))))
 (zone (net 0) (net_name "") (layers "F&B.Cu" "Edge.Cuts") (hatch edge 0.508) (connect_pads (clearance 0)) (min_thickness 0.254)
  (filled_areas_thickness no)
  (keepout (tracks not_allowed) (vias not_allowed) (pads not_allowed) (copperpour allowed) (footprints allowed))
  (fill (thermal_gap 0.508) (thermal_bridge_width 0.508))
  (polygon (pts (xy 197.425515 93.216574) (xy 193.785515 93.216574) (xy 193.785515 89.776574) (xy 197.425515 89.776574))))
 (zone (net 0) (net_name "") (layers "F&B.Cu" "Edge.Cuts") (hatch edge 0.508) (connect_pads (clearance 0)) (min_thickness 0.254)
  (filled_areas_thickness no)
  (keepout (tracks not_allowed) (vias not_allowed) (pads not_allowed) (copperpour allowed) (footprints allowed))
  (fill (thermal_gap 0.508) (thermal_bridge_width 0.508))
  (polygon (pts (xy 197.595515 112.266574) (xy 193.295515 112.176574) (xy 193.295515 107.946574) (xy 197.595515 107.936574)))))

